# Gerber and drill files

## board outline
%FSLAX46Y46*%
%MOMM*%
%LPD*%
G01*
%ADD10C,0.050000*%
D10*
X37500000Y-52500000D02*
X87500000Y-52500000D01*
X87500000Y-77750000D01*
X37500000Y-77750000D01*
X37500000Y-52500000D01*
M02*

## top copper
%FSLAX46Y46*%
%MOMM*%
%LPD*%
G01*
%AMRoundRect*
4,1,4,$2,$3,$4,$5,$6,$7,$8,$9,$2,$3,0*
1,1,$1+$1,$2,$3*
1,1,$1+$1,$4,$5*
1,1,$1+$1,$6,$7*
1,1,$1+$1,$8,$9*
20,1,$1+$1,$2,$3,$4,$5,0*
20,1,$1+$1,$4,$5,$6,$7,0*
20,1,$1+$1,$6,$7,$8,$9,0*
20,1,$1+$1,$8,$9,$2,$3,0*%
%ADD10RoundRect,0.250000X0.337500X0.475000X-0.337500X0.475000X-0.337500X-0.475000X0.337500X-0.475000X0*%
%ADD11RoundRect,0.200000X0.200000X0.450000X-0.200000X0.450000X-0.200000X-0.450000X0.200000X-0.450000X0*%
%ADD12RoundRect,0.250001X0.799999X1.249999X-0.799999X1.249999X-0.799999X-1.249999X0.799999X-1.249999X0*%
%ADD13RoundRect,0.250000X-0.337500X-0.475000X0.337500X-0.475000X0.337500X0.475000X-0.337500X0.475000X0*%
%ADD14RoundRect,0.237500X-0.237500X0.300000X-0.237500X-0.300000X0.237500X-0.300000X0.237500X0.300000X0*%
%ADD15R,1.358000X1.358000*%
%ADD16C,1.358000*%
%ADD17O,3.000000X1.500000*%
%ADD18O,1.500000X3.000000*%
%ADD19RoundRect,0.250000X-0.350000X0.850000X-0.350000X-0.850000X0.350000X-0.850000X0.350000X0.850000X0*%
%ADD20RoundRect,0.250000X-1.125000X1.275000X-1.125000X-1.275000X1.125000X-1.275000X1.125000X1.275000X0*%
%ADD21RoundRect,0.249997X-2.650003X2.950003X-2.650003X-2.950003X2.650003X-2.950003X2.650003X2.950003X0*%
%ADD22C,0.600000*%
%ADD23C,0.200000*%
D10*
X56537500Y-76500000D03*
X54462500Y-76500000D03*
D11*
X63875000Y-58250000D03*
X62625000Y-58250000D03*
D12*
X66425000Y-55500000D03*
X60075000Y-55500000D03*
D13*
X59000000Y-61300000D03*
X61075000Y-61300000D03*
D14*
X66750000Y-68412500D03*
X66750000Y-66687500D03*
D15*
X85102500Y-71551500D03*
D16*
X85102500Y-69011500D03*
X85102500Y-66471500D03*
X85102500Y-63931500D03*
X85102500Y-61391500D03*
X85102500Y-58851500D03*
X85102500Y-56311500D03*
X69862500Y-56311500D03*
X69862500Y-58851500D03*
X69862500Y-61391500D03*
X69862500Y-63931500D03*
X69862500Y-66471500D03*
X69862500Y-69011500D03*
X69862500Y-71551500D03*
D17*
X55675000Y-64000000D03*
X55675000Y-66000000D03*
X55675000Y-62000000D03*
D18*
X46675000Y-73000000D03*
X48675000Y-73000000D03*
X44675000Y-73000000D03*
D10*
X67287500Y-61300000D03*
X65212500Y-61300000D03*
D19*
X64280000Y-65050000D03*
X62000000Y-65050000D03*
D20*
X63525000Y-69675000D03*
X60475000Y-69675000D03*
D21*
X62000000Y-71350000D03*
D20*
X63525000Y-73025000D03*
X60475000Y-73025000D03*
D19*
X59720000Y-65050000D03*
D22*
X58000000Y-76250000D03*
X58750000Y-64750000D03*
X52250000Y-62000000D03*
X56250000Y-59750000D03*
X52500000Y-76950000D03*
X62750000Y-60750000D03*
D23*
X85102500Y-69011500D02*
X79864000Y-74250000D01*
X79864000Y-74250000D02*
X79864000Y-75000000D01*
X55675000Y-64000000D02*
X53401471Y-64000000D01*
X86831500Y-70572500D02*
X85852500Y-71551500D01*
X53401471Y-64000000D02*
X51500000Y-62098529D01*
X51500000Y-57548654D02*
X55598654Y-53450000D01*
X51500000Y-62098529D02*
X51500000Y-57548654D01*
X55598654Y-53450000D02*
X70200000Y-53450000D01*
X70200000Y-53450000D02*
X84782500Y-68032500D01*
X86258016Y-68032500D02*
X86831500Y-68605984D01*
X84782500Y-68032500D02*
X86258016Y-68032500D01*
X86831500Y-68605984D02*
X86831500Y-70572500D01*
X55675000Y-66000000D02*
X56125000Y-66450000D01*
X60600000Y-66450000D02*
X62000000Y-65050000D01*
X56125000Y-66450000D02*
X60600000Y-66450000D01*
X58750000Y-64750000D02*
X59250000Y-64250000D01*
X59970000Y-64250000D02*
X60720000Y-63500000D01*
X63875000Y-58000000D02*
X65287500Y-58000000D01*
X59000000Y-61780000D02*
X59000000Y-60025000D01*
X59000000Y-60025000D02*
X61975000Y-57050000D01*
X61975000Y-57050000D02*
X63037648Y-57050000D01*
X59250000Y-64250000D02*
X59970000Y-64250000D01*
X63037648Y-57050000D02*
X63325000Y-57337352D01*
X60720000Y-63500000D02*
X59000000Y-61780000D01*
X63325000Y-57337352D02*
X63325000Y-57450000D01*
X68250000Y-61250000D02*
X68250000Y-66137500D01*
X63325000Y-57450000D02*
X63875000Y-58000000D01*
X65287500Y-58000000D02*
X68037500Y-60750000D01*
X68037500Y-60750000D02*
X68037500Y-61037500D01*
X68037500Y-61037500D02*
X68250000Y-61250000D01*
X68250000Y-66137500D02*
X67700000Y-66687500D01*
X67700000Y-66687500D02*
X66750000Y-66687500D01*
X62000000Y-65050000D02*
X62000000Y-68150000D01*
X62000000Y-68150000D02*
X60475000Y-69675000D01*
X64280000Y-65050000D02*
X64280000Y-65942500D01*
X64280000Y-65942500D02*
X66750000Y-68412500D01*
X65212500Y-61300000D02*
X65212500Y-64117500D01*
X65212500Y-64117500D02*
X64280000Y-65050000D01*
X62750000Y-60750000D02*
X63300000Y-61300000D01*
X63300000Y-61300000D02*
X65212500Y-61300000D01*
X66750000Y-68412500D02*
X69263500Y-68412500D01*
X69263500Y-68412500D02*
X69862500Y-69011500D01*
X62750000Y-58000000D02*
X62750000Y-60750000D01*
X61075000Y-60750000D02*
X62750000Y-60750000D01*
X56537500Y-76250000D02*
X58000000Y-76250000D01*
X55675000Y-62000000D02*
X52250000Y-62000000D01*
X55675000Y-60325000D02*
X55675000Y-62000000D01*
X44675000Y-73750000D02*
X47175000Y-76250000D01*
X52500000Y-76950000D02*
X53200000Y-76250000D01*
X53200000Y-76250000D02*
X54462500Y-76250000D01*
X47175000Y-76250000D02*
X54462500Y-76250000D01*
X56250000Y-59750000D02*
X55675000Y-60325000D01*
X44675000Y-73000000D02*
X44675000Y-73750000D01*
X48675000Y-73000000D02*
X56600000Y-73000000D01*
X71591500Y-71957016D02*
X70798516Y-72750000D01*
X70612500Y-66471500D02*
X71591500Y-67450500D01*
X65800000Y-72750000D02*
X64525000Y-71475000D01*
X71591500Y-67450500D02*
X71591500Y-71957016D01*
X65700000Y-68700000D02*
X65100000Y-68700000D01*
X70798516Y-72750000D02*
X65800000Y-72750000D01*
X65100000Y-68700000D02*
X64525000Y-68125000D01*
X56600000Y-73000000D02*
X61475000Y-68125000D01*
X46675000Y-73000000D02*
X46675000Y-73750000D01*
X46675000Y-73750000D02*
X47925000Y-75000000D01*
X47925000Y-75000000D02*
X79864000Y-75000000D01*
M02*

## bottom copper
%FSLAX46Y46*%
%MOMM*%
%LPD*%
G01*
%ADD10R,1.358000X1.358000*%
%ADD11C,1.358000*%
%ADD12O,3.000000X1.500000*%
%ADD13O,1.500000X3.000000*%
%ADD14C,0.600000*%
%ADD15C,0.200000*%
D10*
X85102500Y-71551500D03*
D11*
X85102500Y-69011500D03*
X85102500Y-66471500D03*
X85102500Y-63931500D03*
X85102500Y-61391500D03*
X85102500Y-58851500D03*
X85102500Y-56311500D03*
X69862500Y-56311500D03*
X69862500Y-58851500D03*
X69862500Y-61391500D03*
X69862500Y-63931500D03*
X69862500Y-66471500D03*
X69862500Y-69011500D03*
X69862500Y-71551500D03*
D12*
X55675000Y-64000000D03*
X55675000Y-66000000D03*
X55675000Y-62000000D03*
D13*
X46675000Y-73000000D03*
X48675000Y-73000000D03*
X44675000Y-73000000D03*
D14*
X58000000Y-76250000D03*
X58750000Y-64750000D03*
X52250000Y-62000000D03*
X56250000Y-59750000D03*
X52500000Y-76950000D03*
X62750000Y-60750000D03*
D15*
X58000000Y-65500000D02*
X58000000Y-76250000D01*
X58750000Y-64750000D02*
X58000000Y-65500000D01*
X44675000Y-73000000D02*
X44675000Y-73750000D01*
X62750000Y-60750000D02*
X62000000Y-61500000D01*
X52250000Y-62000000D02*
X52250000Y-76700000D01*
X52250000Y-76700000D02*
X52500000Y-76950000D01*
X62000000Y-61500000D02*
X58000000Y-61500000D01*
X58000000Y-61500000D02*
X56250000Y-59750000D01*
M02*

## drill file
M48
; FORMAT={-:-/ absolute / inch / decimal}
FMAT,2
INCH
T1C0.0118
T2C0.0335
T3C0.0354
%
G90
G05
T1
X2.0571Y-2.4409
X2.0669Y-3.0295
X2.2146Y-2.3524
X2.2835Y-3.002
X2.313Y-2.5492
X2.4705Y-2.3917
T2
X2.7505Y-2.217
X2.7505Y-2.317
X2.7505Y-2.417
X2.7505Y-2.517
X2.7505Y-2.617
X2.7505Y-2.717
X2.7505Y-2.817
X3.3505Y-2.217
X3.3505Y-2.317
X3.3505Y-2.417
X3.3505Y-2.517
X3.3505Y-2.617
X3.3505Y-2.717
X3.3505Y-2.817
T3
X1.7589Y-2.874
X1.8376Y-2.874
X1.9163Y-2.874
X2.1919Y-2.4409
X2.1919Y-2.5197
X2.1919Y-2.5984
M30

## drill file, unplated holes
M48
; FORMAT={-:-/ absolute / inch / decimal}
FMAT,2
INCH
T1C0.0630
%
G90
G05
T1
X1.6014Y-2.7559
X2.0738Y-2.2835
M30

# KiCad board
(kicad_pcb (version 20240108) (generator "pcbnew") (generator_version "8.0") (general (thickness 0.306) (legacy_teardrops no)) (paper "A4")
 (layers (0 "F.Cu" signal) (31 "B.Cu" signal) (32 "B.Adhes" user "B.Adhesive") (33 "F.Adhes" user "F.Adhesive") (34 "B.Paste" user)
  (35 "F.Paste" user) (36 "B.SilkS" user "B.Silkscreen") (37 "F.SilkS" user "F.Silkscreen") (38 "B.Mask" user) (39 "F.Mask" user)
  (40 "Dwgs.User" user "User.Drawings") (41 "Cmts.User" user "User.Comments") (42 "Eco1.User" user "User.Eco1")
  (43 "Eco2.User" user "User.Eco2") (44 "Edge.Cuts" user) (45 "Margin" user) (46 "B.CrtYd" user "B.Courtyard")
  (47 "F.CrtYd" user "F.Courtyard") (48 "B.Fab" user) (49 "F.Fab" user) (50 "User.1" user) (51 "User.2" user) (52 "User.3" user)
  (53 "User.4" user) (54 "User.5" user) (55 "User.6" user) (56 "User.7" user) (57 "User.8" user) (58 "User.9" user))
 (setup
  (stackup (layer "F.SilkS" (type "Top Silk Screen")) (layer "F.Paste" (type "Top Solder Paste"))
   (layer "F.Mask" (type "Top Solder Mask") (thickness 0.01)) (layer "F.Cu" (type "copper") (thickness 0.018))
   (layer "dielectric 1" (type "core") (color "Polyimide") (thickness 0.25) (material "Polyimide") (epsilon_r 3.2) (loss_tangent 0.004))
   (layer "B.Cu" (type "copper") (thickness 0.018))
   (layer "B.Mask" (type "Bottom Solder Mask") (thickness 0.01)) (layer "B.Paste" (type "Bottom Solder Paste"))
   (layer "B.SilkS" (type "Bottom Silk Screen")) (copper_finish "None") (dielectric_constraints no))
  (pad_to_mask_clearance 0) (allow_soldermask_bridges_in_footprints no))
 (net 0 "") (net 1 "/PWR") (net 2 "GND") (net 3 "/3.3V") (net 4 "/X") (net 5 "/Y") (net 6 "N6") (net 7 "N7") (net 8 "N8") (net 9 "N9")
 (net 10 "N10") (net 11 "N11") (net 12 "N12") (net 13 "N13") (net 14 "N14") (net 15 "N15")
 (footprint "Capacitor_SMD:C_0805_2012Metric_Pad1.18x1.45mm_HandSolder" (layer "F.Cu") (at 55.5 76.5 180)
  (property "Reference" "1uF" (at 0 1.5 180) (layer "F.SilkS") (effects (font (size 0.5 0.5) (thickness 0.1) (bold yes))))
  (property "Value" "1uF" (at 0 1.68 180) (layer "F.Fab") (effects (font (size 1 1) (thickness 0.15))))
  (pad "1" smd roundrect (at -1.0375 0 180) (size 1.175 1.45) (layers "F.Cu" "F.Paste" "F.Mask") (roundrect_rratio 0.212766) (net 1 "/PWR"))
  (pad "2" smd roundrect (at 1.0375 0 180) (size 1.175 1.45) (layers "F.Cu" "F.Paste" "F.Mask") (roundrect_rratio 0.212766) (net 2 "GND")))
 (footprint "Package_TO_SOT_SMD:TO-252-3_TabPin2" (layer "F.Cu") (at 62 70.09 -90)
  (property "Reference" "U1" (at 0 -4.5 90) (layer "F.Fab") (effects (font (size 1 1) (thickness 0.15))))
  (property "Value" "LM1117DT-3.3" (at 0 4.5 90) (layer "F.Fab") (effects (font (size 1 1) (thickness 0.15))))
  (pad "1" smd roundrect (at -5.04 -2.28 270) (size 2.2 1.2) (layers "F.Cu" "F.Paste" "F.Mask") (roundrect_rratio 0.208333) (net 2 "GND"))
  (pad "2" smd roundrect (at -5.04 0 270) (size 2.2 1.2) (layers "F.Cu" "F.Paste" "F.Mask") (roundrect_rratio 0.208333) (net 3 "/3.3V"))
  (pad "2" smd roundrect (at -0.415 -1.525 270) (size 3.05 2.75) (layers "F.Cu" "F.Paste") (roundrect_rratio 0.090909) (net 3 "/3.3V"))
  (pad "2" smd roundrect (at -0.415 1.525 270) (size 3.05 2.75) (layers "F.Cu" "F.Paste") (roundrect_rratio 0.090909) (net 3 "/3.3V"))
  (pad "2" smd roundrect (at 1.26 0 270) (size 6.4 5.8) (layers "F.Cu" "F.Mask") (roundrect_rratio 0.043103) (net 3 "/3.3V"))
  (pad "2" smd roundrect (at 2.935 -1.525 270) (size 3.05 2.75) (layers "F.Cu" "F.Paste") (roundrect_rratio 0.090909) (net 3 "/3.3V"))
  (pad "2" smd roundrect (at 2.935 1.525 270) (size 3.05 2.75) (layers "F.Cu" "F.Paste") (roundrect_rratio 0.090909) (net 3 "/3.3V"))
  (pad "3" smd roundrect (at -5.04 2.28 270) (size 2.2 1.2) (layers "F.Cu" "F.Paste" "F.Mask") (roundrect_rratio 0.208333) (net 1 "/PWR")))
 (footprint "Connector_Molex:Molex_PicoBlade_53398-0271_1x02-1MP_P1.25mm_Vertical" (layer "F.Cu") (at 63.25 57 180)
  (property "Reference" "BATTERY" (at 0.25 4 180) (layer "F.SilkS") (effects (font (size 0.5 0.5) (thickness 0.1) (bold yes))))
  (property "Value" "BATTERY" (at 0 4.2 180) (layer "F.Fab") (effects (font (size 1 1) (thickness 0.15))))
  (pad "1" smd roundrect (at -0.625 -1.25 180) (size 0.8 1.3) (layers "F.Cu" "F.Paste" "F.Mask") (roundrect_rratio 0.25) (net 1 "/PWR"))
  (pad "2" smd roundrect (at 0.625 -1.25 180) (size 0.8 1.3) (layers "F.Cu" "F.Paste" "F.Mask") (roundrect_rratio 0.25) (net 2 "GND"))
  (pad "MP" smd roundrect (at -3.175 1.5 180) (size 2.1 3) (layers "F.Cu" "F.Paste" "F.Mask") (roundrect_rratio 0.119048))
  (pad "MP" smd roundrect (at 3.175 1.5 180) (size 2.1 3) (layers "F.Cu" "F.Paste" "F.Mask") (roundrect_rratio 0.119048)))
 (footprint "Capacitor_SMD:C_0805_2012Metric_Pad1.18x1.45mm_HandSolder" (layer "F.Cu") (at 60.0375 61.3)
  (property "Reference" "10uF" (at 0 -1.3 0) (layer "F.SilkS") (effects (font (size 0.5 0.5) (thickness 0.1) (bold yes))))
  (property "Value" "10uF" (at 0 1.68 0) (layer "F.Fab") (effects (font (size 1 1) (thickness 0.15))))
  (pad "1" smd roundrect (at -1.0375 0) (size 1.175 1.45) (layers "F.Cu" "F.Paste" "F.Mask") (roundrect_rratio 0.212766) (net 1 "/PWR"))
  (pad "2" smd roundrect (at 1.0375 0) (size 1.175 1.45) (layers "F.Cu" "F.Paste" "F.Mask") (roundrect_rratio 0.212766) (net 2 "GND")))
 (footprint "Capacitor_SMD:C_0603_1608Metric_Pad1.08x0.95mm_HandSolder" (layer "F.Cu") (at 66.75 67.55 -90)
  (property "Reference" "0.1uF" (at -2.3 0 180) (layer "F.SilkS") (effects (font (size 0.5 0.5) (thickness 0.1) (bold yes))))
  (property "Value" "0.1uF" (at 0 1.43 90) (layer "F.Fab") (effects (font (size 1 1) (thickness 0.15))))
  (pad "1" smd roundrect (at -0.8625 0 270) (size 1.075 0.95) (layers "F.Cu" "F.Paste" "F.Mask") (roundrect_rratio 0.25) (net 1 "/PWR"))
  (pad "2" smd roundrect (at 0.8625 0 270) (size 1.075 0.95) (layers "F.Cu" "F.Paste" "F.Mask") (roundrect_rratio 0.25) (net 2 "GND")))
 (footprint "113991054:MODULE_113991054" (layer "F.Cu") (at 77.4825 63.995 180)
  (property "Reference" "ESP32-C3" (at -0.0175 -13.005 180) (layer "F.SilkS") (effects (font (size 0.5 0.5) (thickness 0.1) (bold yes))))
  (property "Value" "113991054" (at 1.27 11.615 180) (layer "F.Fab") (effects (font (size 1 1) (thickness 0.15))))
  (pad "1" thru_hole rect (at -7.62 -7.5565 180) (size 1.358 1.358) (drill 0.85) (layers "*.Cu" "*.Mask") (remove_unused_layers no)
   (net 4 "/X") (solder_mask_margin 0.102))
  (pad "2" thru_hole circle (at -7.62 -5.0165 180) (size 1.358 1.358) (drill 0.85) (layers "*.Cu" "*.Mask") (remove_unused_layers no)
   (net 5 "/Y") (solder_mask_margin 0.102))
  (pad "3" thru_hole circle (at -7.62 -2.4765 180) (size 1.358 1.358) (drill 0.85) (layers "*.Cu" "*.Mask") (remove_unused_layers no)
   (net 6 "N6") (solder_mask_margin 0.102))
  (pad "4" thru_hole circle (at -7.62 0.0635 180) (size 1.358 1.358) (drill 0.85) (layers "*.Cu" "*.Mask") (remove_unused_layers no)
   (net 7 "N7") (solder_mask_margin 0.102))
  (pad "5" thru_hole circle (at -7.62 2.6035 180) (size 1.358 1.358) (drill 0.85) (layers "*.Cu" "*.Mask") (remove_unused_layers no)
   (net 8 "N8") (solder_mask_margin 0.102))
  (pad "6" thru_hole circle (at -7.62 5.1435 180) (size 1.358 1.358) (drill 0.85) (layers "*.Cu" "*.Mask") (remove_unused_layers no)
   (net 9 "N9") (solder_mask_margin 0.102))
  (pad "7" thru_hole circle (at -7.62 7.6835 180) (size 1.358 1.358) (drill 0.85) (layers "*.Cu" "*.Mask") (remove_unused_layers no)
   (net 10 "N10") (solder_mask_margin 0.102))
  (pad "8" thru_hole circle (at 7.62 7.6835 180) (size 1.358 1.358) (drill 0.85) (layers "*.Cu" "*.Mask") (remove_unused_layers no)
   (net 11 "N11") (solder_mask_margin 0.102))
  (pad "9" thru_hole circle (at 7.62 5.1435 180) (size 1.358 1.358) (drill 0.85) (layers "*.Cu" "*.Mask") (remove_unused_layers no)
   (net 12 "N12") (solder_mask_margin 0.102))
  (pad "10" thru_hole circle (at 7.62 2.6035 180) (size 1.358 1.358) (drill 0.85) (layers "*.Cu" "*.Mask") (remove_unused_layers no)
   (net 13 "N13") (solder_mask_margin 0.102))
  (pad "11" thru_hole circle (at 7.62 0.0635 180) (size 1.358 1.358) (drill 0.85) (layers "*.Cu" "*.Mask") (remove_unused_layers no)
   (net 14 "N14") (solder_mask_margin 0.102))
  (pad "12" thru_hole circle (at 7.62 -2.4765 180) (size 1.358 1.358) (drill 0.85) (layers "*.Cu" "*.Mask") (remove_unused_layers no)
   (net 3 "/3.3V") (solder_mask_margin 0.102))
  (pad "13" thru_hole circle (at 7.62 -5.0165 180) (size 1.358 1.358) (drill 0.85) (layers "*.Cu" "*.Mask") (remove_unused_layers no)
   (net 2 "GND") (solder_mask_margin 0.102))
  (pad "14" thru_hole circle (at 7.62 -7.5565 180) (size 1.358 1.358) (drill 0.85) (layers "*.Cu" "*.Mask") (remove_unused_layers no)
   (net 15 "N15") (solder_mask_margin 0.102)))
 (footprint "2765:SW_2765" (layer "F.Cu") (at 46.675 64)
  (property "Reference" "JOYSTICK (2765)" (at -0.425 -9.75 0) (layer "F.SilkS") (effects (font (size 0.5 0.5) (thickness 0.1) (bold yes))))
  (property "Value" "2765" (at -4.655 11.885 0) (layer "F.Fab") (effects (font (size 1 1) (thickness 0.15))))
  (pad "" np_thru_hole circle (at -6 6) (size 1.6 1.6) (drill 1.6) (layers "*.Cu" "*.Mask"))
  (pad "" np_thru_hole circle (at 6 -6) (size 1.6 1.6) (drill 1.6) (layers "*.Cu" "*.Mask"))
  (pad "X" thru_hole oval (at 9 0) (size 3 1.5) (drill 0.9) (layers "*.Cu" "*.Mask") (remove_unused_layers no) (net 4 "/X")
   (solder_mask_margin 0.102))
  (pad "X+" thru_hole oval (at 9 2) (size 3 1.5) (drill 0.9) (layers "*.Cu" "*.Mask") (remove_unused_layers no) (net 3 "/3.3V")
   (solder_mask_margin 0.102))
  (pad "X-" thru_hole oval (at 9 -2) (size 3 1.5) (drill 0.9) (layers "*.Cu" "*.Mask") (remove_unused_layers no) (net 2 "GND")
   (solder_mask_margin 0.102))
  (pad "Y" thru_hole oval (at 0 9) (size 1.5 3) (drill 0.9) (layers "*.Cu" "*.Mask") (remove_unused_layers no) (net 5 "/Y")
   (solder_mask_margin 0.102))
  (pad "Y+" thru_hole oval (at 2 9) (size 1.5 3) (drill 0.9) (layers "*.Cu" "*.Mask") (remove_unused_layers no) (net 3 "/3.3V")
   (solder_mask_margin 0.102))
  (pad "Y-" thru_hole oval (at -2 9) (size 1.5 3) (drill 0.9) (layers "*.Cu" "*.Mask") (remove_unused_layers no) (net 2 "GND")
   (solder_mask_margin 0.102)))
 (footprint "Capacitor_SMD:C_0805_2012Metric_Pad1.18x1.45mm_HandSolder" (layer "F.Cu") (at 66.25 61.3 180)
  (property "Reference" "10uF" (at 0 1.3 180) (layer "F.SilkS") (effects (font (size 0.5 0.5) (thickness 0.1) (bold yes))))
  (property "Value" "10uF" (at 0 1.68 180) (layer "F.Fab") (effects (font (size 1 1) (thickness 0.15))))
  (pad "1" smd roundrect (at -1.0375 0 180) (size 1.175 1.45) (layers "F.Cu" "F.Paste" "F.Mask") (roundrect_rratio 0.212766) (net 1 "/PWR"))
  (pad "2" smd roundrect (at 1.0375 0 180) (size 1.175 1.45) (layers "F.Cu" "F.Paste" "F.Mask") (roundrect_rratio 0.212766) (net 2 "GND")))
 (gr_rect (start 37.5 52.5) (end 87.5 77.75) (stroke (width 0.05) (type default)) (fill none) (layer "Edge.Cuts"))
 (segment (start 61.975 57.05) (end 63.037648 57.05) (width 0.2) (layer "F.Cu") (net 1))
 (segment (start 63.325 57.337352) (end 63.325 57.45) (width 0.2) (layer "F.Cu") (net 1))
 (segment (start 63.037648 57.05) (end 63.325 57.337352) (width 0.2) (layer "F.Cu") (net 1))
 (segment (start 59 60.025) (end 61.975 57.05) (width 0.2) (layer "F.Cu") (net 1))
 (segment (start 63.875 58) (end 65.2875 58) (width 0.2) (layer "F.Cu") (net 1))
 (segment (start 60.72 63.5) (end 59 61.78) (width 0.2) (layer "F.Cu") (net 1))
 (segment (start 63.325 57.45) (end 63.875 58) (width 0.2) (layer "F.Cu") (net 1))
 (segment (start 68.0375 61.0375) (end 68.25 61.25) (width 0.2) (layer "F.Cu") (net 1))
 (segment (start 58.75 64.75) (end 59.25 64.25) (width 0.2) (layer "F.Cu") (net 1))
 (segment (start 65.2875 58) (end 68.0375 60.75) (width 0.2) (layer "F.Cu") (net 1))
 (segment (start 59.25 64.25) (end 59.97 64.25) (width 0.2) (layer "F.Cu") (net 1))
 (segment (start 67.7 66.6875) (end 66.75 66.6875) (width 0.2) (layer "F.Cu") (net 1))
 (segment (start 68.0375 60.75) (end 68.0375 61.0375) (width 0.2) (layer "F.Cu") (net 1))
 (segment (start 68.25 61.25) (end 68.25 66.1375) (width 0.2) (layer "F.Cu") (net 1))
 (segment (start 59 61.78) (end 59 60.025) (width 0.2) (layer "F.Cu") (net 1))
 (segment (start 56.5375 76.25) (end 58 76.25) (width 0.2) (layer "F.Cu") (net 1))
 (segment (start 59.97 64.25) (end 60.72 63.5) (width 0.2) (layer "F.Cu") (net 1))
 (segment (start 68.25 66.1375) (end 67.7 66.6875) (width 0.2) (layer "F.Cu") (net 1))
 (via (at 58 76.25) (size 0.6) (drill 0.3) (layers "F.Cu" "B.Cu") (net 1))
 (via (at 58.75 64.75) (size 0.6) (drill 0.3) (layers "F.Cu" "B.Cu") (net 1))
 (segment (start 58 65.5) (end 58 76.25) (width 0.2) (layer "B.Cu") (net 1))
 (segment (start 58.75 64.75) (end 58 65.5) (width 0.2) (layer "B.Cu") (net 1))
 (segment (start 55.675 62) (end 52.25 62) (width 0.2) (layer "F.Cu") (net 2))
 (segment (start 64.28 65.9425) (end 66.75 68.4125) (width 0.2) (layer "F.Cu") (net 2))
 (segment (start 55.675 60.325) (end 55.675 62) (width 0.2) (layer "F.Cu") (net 2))
 (segment (start 61.075 60.75) (end 62.75 60.75) (width 0.2) (layer "F.Cu") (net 2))
 (segment (start 69.2635 68.4125) (end 69.8625 69.0115) (width 0.2) (layer "F.Cu") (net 2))
 (segment (start 44.675 73.75) (end 47.175 76.25) (width 0.2) (layer "F.Cu") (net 2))
 (segment (start 62.75 60.75) (end 63.3 61.3) (width 0.2) (layer "F.Cu") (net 2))
 (segment (start 52.5 76.95) (end 53.2 76.25) (width 0.2) (layer "F.Cu") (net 2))
 (segment (start 62.75 58) (end 62.75 60.75) (width 0.2) (layer "F.Cu") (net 2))
 (segment (start 53.2 76.25) (end 54.4625 76.25) (width 0.2) (layer "F.Cu") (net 2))
 (segment (start 65.2125 61.3) (end 65.2125 64.1175) (width 0.2) (layer "F.Cu") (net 2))
 (segment (start 66.75 68.4125) (end 69.2635 68.4125) (width 0.2) (layer "F.Cu") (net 2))
 (segment (start 65.2125 64.1175) (end 64.28 65.05) (width 0.2) (layer "F.Cu") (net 2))
 (segment (start 47.175 76.25) (end 54.4625 76.25) (width 0.2) (layer "F.Cu") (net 2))
 (segment (start 63.3 61.3) (end 65.2125 61.3) (width 0.2) (layer "F.Cu") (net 2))
 (segment (start 64.28 65.05) (end 64.28 65.9425) (width 0.2) (layer "F.Cu") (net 2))
 (segment (start 56.25 59.75) (end 55.675 60.325) (width 0.2) (layer "F.Cu") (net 2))
 (segment (start 44.675 73) (end 44.675 73.75) (width 0.2) (layer "F.Cu") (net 2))
 (via (at 52.25 62) (size 0.6) (drill 0.3) (layers "F.Cu" "B.Cu") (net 2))
 (via (at 56.25 59.75) (size 0.6) (drill 0.3) (layers "F.Cu" "B.Cu") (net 2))
 (via (at 52.5 76.95) (size 0.6) (drill 0.3) (layers "F.Cu" "B.Cu") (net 2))
 (via (at 62.75 60.75) (size 0.6) (drill 0.3) (layers "F.Cu" "B.Cu") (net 2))
 (segment (start 44.675 73) (end 44.675 73.75) (width 0.2) (layer "B.Cu") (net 2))
 (segment (start 62.75 60.75) (end 62 61.5) (width 0.2) (layer "B.Cu") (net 2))
 (segment (start 52.25 62) (end 52.25 76.7) (width 0.2) (layer "B.Cu") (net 2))
 (segment (start 52.25 76.7) (end 52.5 76.95) (width 0.2) (layer "B.Cu") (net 2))
 (segment (start 62 61.5) (end 58 61.5) (width 0.2) (layer "B.Cu") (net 2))
 (segment (start 58 61.5) (end 56.25 59.75) (width 0.2) (layer "B.Cu") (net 2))
 (segment (start 56.125 66.45) (end 60.6 66.45) (width 0.2) (layer "F.Cu") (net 3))
 (segment (start 48.675 73) (end 56.6 73) (width 0.2) (layer "F.Cu") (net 3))
 (segment (start 71.5915 71.957016) (end 70.798516 72.75) (width 0.2) (layer "F.Cu") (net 3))
 (segment (start 70.6125 66.4715) (end 71.5915 67.4505) (width 0.2) (layer "F.Cu") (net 3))
 (segment (start 55.675 66) (end 56.125 66.45) (width 0.2) (layer "F.Cu") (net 3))
 (segment (start 65.8 72.75) (end 64.525 71.475) (width 0.2) (layer "F.Cu") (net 3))
 (segment (start 71.5915 67.4505) (end 71.5915 71.957016) (width 0.2) (layer "F.Cu") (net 3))
 (segment (start 65.7 68.7) (end 65.1 68.7) (width 0.2) (layer "F.Cu") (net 3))
 (segment (start 70.798516 72.75) (end 65.8 72.75) (width 0.2) (layer "F.Cu") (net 3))
 (segment (start 62 65.05) (end 62 68.15) (width 0.2) (layer "F.Cu") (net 3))
 (segment (start 65.1 68.7) (end 64.525 68.125) (width 0.2) (layer "F.Cu") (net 3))
 (segment (start 60.6 66.45) (end 62 65.05) (width 0.2) (layer "F.Cu") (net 3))
 (segment (start 56.6 73) (end 61.475 68.125) (width 0.2) (layer "F.Cu") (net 3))
 (segment (start 62 68.15) (end 60.475 69.675) (width 0.2) (layer "F.Cu") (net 3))
 (segment (start 46.675 73) (end 46.675 73.75) (width 0.2) (layer "F.Cu") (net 5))
 (segment (start 46.675 73.75) (end 47.925 75) (width 0.2) (layer "F.Cu") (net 5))
 (segment (start 85.1025 69.0115) (end 79.864 74.25) (width 0.2) (layer "F.Cu") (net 5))
 (segment (start 47.925 75) (end 79.864 75) (width 0.2) (layer "F.Cu") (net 5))
 (segment (start 79.864 74.25) (end 79.864 75) (width 0.2) (layer "F.Cu") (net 5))
 (segment (start 86.8315 70.5725) (end 85.8525 71.5515) (width 0.2) (layer "F.Cu") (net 4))
 (segment (start 51.5 62.098529) (end 51.5 57.548654) (width 0.2) (layer "F.Cu") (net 4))
 (segment (start 51.5 57.548654) (end 55.598654 53.45) (width 0.2) (layer "F.Cu") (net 4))
 (segment (start 55.598654 53.45) (end 70.2 53.45) (width 0.2) (layer "F.Cu") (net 4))
 (segment (start 86.258016 68.0325) (end 86.8315 68.605984) (width 0.2) (layer "F.Cu") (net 4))
 (segment (start 70.2 53.45) (end 84.7825 68.0325) (width 0.2) (layer "F.Cu") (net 4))
 (segment (start 84.7825 68.0325) (end 86.258016 68.0325) (width 0.2) (layer "F.Cu") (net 4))
 (segment (start 55.675 64) (end 53.401471 64) (width 0.2) (layer "F.Cu") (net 4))
 (segment (start 53.401471 64) (end 51.5 62.098529) (width 0.2) (layer "F.Cu") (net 4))
 (segment (start 86.8315 68.605984) (end 86.8315 70.5725) (width 0.2) (layer "F.Cu") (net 4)))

